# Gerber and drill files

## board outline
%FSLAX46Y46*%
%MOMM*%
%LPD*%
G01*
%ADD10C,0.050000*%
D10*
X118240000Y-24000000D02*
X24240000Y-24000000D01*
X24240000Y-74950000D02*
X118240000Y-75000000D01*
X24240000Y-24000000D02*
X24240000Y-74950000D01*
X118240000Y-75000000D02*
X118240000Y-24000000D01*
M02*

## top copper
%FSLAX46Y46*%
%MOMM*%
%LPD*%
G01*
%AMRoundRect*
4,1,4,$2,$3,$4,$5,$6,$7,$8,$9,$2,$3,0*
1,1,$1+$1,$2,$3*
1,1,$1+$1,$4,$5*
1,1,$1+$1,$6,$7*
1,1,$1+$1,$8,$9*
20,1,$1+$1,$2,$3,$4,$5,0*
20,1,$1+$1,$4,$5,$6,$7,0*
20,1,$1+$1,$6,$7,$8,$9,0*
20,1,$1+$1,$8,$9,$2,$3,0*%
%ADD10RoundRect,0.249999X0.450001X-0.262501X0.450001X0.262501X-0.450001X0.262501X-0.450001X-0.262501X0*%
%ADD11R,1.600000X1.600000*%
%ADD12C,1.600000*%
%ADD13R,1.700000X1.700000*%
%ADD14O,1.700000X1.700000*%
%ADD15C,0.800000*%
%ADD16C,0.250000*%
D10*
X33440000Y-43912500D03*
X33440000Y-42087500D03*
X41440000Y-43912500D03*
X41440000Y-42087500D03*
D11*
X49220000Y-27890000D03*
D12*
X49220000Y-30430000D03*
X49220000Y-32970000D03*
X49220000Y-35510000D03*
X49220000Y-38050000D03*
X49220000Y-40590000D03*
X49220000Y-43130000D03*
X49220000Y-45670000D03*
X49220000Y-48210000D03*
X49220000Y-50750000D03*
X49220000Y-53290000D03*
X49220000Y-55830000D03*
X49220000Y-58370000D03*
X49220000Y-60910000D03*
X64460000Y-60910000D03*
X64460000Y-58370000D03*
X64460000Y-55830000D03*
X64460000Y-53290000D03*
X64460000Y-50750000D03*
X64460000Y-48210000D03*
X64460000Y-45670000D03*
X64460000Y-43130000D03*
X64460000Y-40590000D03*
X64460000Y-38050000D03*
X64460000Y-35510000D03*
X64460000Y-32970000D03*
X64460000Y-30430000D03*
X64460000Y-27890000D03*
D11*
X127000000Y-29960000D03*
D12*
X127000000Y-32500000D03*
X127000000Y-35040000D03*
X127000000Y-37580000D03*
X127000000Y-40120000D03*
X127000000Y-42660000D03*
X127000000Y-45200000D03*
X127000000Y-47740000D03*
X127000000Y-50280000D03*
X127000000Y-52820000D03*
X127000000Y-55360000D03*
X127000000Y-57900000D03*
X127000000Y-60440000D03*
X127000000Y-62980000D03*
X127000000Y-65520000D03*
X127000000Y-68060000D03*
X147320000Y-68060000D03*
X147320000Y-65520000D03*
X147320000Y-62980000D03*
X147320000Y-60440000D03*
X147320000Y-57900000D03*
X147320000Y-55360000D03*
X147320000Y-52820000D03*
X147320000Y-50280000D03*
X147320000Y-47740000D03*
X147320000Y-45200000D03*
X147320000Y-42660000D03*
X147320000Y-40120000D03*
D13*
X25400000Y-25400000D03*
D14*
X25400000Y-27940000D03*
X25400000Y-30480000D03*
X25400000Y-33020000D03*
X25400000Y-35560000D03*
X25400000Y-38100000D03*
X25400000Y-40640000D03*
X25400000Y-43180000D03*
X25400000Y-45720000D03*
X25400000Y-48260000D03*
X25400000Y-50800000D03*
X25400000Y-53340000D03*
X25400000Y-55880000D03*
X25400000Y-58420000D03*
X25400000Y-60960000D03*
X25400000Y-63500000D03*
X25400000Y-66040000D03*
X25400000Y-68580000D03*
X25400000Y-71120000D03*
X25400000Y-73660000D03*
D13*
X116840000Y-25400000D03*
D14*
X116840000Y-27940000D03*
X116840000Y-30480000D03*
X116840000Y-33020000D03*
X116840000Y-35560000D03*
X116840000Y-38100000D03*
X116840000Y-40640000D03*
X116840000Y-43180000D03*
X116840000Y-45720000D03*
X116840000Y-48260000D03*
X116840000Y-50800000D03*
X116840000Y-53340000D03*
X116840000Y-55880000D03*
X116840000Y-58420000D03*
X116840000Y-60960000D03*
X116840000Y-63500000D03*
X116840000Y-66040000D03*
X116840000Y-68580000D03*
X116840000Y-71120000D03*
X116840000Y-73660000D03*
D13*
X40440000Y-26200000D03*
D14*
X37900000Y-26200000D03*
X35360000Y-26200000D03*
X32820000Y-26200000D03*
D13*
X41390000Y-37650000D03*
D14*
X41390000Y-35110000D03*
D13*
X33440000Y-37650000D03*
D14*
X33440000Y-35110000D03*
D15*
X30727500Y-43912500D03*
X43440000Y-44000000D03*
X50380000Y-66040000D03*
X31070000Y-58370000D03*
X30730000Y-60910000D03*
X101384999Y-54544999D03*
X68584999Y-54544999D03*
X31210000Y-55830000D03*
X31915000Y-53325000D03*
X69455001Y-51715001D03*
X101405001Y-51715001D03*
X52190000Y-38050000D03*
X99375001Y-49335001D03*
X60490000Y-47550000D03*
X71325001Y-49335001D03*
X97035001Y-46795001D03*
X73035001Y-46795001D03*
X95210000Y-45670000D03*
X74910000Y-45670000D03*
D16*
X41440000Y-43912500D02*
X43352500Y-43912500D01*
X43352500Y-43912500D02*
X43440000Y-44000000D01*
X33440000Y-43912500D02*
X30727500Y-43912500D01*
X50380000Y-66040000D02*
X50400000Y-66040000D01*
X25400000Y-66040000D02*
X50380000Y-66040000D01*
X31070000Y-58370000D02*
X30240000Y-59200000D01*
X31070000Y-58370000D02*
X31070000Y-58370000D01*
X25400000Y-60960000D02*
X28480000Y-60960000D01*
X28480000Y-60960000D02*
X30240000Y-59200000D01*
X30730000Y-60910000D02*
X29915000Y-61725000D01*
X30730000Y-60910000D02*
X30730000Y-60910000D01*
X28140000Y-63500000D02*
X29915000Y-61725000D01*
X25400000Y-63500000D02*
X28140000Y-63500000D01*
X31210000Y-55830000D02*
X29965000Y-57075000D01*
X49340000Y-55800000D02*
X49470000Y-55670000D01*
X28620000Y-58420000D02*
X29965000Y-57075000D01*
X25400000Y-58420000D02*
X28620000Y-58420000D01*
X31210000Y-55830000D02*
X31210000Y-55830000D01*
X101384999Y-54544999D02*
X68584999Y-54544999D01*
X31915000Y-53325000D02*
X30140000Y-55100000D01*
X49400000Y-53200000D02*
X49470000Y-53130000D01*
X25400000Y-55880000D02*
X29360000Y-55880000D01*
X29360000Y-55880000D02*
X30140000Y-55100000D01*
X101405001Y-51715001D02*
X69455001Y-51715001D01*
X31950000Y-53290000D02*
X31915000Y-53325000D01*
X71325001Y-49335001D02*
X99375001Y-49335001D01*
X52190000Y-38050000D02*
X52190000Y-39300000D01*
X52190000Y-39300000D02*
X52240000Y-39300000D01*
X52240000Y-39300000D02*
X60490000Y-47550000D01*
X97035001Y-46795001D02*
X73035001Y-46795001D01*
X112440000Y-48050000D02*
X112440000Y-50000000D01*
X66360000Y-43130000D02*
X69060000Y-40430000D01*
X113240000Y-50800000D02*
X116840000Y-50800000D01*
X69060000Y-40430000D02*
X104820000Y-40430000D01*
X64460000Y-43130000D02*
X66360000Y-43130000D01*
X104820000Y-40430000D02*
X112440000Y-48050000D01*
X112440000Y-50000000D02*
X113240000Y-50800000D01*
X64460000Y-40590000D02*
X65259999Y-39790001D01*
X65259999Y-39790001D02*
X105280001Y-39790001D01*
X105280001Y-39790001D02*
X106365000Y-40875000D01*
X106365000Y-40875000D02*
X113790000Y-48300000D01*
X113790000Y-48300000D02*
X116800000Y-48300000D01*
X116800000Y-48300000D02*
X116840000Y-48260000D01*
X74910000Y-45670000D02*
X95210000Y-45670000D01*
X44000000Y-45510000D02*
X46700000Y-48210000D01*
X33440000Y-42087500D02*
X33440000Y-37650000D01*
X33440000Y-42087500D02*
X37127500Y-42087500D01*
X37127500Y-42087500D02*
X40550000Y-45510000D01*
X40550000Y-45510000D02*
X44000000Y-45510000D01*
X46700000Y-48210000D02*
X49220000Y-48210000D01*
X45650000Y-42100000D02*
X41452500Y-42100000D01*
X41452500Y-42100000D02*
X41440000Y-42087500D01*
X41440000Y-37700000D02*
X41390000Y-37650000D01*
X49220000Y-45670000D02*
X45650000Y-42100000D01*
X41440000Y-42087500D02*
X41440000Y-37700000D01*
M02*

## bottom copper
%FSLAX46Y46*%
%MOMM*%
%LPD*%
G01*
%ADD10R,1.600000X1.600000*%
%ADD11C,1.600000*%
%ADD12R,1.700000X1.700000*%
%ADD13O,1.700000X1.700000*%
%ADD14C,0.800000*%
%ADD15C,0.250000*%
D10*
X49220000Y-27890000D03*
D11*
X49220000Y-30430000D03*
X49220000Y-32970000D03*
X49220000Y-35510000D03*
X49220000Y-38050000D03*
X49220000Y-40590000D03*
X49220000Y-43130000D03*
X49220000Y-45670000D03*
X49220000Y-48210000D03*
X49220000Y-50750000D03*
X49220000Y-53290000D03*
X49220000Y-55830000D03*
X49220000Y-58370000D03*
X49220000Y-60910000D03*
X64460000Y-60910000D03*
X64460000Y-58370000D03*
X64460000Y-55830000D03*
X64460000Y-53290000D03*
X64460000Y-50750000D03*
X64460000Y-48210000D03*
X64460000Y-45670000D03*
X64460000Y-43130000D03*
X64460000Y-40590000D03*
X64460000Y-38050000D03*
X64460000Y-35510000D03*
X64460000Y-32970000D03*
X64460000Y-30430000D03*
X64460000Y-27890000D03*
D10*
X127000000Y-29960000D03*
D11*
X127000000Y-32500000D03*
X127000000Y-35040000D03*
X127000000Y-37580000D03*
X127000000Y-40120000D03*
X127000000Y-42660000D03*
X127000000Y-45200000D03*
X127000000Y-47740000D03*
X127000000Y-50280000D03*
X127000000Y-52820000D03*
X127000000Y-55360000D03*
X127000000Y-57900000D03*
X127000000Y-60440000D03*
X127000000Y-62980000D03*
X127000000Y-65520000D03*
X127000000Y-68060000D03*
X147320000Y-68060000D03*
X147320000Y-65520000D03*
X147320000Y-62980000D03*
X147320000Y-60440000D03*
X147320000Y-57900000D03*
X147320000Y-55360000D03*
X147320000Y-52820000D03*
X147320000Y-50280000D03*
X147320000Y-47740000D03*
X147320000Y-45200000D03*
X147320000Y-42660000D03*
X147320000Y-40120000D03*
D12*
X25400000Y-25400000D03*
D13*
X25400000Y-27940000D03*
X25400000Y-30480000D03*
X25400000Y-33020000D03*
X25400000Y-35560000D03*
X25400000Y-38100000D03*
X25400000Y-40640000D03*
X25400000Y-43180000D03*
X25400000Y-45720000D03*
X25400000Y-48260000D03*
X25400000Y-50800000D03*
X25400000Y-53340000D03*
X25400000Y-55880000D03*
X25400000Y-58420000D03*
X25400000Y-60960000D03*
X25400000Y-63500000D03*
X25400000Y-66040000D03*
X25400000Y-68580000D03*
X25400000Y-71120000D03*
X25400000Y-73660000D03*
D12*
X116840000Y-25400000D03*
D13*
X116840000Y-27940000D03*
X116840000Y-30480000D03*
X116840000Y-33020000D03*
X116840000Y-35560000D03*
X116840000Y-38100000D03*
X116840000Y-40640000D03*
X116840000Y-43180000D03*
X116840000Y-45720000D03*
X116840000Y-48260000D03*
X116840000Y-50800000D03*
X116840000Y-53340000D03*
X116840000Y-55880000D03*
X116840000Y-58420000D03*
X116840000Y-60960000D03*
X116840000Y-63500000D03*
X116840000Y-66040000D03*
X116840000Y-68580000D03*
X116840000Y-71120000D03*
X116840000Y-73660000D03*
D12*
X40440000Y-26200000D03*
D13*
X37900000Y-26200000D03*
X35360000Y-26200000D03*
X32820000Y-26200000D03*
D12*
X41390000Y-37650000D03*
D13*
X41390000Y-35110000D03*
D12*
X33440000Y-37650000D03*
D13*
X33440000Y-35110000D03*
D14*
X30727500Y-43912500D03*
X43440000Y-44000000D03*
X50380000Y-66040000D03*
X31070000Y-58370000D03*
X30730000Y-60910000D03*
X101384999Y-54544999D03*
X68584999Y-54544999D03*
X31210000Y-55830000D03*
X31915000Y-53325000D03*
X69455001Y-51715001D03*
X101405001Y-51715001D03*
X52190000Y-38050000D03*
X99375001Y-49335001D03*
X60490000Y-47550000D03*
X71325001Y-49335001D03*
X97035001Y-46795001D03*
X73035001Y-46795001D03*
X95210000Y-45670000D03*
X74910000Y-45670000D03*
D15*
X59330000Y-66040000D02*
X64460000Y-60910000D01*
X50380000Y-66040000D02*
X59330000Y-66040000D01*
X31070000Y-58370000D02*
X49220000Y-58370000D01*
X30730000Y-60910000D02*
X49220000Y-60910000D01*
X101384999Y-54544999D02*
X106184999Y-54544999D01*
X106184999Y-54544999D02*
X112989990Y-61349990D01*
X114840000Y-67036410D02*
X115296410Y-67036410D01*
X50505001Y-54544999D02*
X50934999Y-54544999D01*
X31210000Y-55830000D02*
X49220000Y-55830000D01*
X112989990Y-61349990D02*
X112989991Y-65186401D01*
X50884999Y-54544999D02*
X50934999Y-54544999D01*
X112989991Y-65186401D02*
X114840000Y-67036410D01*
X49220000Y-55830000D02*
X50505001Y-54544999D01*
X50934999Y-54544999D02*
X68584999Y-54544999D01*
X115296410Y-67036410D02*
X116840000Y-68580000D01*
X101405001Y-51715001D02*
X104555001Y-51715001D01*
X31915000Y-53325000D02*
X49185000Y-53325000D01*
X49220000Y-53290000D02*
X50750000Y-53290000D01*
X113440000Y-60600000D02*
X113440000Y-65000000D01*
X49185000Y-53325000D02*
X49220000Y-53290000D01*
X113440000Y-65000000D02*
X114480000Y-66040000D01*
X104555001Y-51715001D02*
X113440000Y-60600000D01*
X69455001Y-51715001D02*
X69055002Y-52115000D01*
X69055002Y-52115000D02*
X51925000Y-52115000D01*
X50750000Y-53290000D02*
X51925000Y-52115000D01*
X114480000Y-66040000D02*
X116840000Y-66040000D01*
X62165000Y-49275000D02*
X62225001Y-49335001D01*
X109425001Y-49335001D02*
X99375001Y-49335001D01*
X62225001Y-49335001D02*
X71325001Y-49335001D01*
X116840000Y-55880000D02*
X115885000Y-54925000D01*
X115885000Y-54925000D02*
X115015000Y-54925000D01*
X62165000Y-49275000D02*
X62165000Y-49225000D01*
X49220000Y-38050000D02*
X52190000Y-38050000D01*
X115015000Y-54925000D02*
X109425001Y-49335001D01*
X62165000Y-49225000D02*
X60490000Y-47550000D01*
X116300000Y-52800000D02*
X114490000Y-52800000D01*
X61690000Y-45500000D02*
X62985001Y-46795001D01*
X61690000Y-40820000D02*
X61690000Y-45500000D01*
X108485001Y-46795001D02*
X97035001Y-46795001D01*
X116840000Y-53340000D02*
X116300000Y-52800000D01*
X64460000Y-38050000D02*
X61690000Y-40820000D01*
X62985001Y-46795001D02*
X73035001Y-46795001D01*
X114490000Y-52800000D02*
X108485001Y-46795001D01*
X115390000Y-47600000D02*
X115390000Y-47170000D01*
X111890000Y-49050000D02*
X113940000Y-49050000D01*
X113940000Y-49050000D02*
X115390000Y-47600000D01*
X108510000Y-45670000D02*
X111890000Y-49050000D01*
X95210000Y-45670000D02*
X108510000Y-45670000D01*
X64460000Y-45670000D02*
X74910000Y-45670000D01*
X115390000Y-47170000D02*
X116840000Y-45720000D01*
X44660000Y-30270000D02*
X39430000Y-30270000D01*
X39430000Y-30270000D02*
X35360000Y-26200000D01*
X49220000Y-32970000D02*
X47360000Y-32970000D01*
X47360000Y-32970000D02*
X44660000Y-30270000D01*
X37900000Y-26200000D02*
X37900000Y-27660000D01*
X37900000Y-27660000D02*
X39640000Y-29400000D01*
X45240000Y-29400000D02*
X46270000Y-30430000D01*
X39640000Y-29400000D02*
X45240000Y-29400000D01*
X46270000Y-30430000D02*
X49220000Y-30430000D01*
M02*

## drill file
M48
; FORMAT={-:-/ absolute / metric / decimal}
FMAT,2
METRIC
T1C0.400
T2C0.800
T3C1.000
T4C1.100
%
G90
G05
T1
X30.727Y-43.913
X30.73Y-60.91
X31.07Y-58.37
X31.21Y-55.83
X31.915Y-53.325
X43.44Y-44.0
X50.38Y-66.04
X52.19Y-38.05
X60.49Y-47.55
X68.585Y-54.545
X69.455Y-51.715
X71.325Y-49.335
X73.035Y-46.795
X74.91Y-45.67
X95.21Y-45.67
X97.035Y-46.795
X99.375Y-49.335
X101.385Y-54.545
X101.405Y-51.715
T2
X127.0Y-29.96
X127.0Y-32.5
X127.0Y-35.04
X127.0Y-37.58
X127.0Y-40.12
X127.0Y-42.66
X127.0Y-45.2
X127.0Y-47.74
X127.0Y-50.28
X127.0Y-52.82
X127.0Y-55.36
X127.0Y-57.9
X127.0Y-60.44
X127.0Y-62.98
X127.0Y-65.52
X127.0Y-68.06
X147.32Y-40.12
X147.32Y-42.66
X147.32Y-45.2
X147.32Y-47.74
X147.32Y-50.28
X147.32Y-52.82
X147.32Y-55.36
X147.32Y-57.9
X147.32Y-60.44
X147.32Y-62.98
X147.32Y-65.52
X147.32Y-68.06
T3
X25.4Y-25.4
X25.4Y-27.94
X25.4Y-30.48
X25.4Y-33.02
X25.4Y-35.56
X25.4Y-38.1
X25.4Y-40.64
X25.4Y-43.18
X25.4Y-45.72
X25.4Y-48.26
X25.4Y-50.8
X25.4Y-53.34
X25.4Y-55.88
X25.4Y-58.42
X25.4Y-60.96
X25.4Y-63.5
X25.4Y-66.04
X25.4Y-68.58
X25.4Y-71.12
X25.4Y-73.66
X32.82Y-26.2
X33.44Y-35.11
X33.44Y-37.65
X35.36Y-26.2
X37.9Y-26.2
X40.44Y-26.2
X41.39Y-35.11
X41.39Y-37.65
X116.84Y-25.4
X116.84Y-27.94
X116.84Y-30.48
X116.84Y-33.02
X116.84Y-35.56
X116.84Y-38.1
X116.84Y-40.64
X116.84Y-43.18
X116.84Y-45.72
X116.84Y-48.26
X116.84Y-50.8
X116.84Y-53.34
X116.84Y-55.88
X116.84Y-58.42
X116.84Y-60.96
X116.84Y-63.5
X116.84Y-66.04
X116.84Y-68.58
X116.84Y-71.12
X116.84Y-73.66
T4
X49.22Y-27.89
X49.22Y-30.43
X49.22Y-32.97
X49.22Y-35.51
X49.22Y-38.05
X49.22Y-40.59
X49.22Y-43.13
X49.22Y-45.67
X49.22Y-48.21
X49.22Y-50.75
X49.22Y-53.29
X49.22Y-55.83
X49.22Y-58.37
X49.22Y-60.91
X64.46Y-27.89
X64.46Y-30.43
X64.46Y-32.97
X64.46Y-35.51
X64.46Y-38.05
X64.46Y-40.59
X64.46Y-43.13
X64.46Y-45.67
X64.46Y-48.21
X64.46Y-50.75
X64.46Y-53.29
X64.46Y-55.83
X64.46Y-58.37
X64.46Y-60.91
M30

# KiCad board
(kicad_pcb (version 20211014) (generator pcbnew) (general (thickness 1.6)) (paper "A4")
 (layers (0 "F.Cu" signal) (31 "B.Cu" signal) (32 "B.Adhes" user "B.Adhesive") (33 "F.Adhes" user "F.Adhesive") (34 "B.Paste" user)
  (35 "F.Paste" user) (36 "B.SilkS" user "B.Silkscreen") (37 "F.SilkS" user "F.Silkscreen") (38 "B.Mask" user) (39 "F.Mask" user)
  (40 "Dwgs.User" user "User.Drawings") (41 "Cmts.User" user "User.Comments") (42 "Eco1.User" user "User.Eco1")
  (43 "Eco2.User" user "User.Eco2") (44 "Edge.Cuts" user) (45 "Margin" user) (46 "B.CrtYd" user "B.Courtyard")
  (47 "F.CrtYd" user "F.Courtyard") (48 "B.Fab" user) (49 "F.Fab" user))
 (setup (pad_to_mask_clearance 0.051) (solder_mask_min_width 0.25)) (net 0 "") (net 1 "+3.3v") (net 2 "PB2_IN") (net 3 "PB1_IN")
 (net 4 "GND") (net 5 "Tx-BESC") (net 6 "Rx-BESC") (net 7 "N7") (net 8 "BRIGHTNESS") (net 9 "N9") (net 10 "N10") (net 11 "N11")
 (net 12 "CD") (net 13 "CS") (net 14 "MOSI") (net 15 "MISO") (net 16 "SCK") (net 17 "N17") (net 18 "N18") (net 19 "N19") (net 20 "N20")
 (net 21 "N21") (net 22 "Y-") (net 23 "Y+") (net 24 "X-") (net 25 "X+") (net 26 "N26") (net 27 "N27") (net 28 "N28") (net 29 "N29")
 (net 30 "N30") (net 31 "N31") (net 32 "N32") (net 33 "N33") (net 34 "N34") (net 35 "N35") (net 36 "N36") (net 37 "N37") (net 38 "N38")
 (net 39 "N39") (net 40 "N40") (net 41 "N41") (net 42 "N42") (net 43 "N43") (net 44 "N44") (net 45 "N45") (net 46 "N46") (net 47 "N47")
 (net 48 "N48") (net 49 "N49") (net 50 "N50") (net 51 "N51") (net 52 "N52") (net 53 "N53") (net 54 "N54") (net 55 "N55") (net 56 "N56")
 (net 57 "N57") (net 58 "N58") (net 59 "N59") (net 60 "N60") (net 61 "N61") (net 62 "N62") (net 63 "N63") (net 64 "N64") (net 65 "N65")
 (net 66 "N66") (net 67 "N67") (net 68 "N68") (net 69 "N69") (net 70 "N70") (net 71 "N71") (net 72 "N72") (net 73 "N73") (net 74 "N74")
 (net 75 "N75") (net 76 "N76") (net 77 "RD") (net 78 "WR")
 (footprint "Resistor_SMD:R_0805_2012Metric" (layer "F.Cu") (at 33.44 43 90)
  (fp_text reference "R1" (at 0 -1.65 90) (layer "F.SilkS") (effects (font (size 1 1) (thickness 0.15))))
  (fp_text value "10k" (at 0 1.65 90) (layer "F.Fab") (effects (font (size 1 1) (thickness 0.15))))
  (pad "1" smd roundrect locked (at -0.9125 0 90) (size 1.025 1.4) (layers "F.Cu" "F.Paste" "F.Mask") (roundrect_rratio 0.2439014634)
   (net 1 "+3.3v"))
  (pad "2" smd roundrect locked (at 0.9125 0 90) (size 1.025 1.4) (layers "F.Cu" "F.Paste" "F.Mask") (roundrect_rratio 0.2439014634)
   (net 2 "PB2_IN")))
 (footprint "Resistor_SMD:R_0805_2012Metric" (layer "F.Cu") (at 41.44 43 90)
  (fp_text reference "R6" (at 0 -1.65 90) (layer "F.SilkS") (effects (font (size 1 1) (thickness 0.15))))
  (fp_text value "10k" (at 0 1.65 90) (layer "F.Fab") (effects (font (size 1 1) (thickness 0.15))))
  (pad "1" smd roundrect locked (at -0.9125 0 90) (size 1.025 1.4) (layers "F.Cu" "F.Paste" "F.Mask") (roundrect_rratio 0.2439014634)
   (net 1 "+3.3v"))
  (pad "2" smd roundrect locked (at 0.9125 0 90) (size 1.025 1.4) (layers "F.Cu" "F.Paste" "F.Mask") (roundrect_rratio 0.2439014634)
   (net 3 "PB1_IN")))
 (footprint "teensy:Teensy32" (layer "F.Cu") (at 56.84 44.4 -90)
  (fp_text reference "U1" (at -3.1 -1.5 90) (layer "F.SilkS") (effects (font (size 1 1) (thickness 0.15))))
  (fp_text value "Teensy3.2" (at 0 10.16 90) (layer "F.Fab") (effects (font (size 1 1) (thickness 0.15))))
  (pad "1" thru_hole rect locked (at -16.51 7.62 270) (size 1.6 1.6) (drill 1.1) (layers *.Cu *.Mask) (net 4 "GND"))
  (pad "2" thru_hole circle locked (at -13.97 7.62 270) (size 1.6 1.6) (drill 1.1) (layers *.Cu *.Mask) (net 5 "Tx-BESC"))
  (pad "3" thru_hole circle locked (at -11.43 7.62 270) (size 1.6 1.6) (drill 1.1) (layers *.Cu *.Mask) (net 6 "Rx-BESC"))
  (pad "4" thru_hole circle locked (at -8.89 7.62 270) (size 1.6 1.6) (drill 1.1) (layers *.Cu *.Mask) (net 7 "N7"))
  (pad "5" thru_hole circle locked (at -6.35 7.62 270) (size 1.6 1.6) (drill 1.1) (layers *.Cu *.Mask) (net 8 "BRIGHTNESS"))
  (pad "6" thru_hole circle locked (at -3.81 7.62 270) (size 1.6 1.6) (drill 1.1) (layers *.Cu *.Mask) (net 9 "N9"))
  (pad "7" thru_hole circle locked (at -1.27 7.62 270) (size 1.6 1.6) (drill 1.1) (layers *.Cu *.Mask) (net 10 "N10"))
  (pad "8" thru_hole circle locked (at 1.27 7.62 270) (size 1.6 1.6) (drill 1.1) (layers *.Cu *.Mask) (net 3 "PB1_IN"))
  (pad "9" thru_hole circle locked (at 3.81 7.62 270) (size 1.6 1.6) (drill 1.1) (layers *.Cu *.Mask) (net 2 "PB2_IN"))
  (pad "10" thru_hole circle locked (at 6.35 7.62 270) (size 1.6 1.6) (drill 1.1) (layers *.Cu *.Mask) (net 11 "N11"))
  (pad "11" thru_hole circle locked (at 8.89 7.62 270) (size 1.6 1.6) (drill 1.1) (layers *.Cu *.Mask) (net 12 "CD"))
  (pad "12" thru_hole circle locked (at 11.43 7.62 270) (size 1.6 1.6) (drill 1.1) (layers *.Cu *.Mask) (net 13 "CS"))
  (pad "13" thru_hole circle locked (at 13.97 7.62 270) (size 1.6 1.6) (drill 1.1) (layers *.Cu *.Mask) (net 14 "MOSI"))
  (pad "14" thru_hole circle locked (at 16.51 7.62 270) (size 1.6 1.6) (drill 1.1) (layers *.Cu *.Mask) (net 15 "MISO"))
  (pad "20" thru_hole circle locked (at 16.51 -7.62 270) (size 1.6 1.6) (drill 1.1) (layers *.Cu *.Mask) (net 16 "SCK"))
  (pad "21" thru_hole circle locked (at 13.97 -7.62 270) (size 1.6 1.6) (drill 1.1) (layers *.Cu *.Mask) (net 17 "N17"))
  (pad "22" thru_hole circle locked (at 11.43 -7.62 270) (size 1.6 1.6) (drill 1.1) (layers *.Cu *.Mask) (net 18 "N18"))
  (pad "23" thru_hole circle locked (at 8.89 -7.62 270) (size 1.6 1.6) (drill 1.1) (layers *.Cu *.Mask) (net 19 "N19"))
  (pad "24" thru_hole circle locked (at 6.35 -7.62 270) (size 1.6 1.6) (drill 1.1) (layers *.Cu *.Mask) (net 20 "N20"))
  (pad "25" thru_hole circle locked (at 3.81 -7.62 270) (size 1.6 1.6) (drill 1.1) (layers *.Cu *.Mask) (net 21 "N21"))
  (pad "26" thru_hole circle locked (at 1.27 -7.62 270) (size 1.6 1.6) (drill 1.1) (layers *.Cu *.Mask) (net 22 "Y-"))
  (pad "27" thru_hole circle locked (at -1.27 -7.62 270) (size 1.6 1.6) (drill 1.1) (layers *.Cu *.Mask) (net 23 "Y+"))
  (pad "28" thru_hole circle locked (at -3.81 -7.62 270) (size 1.6 1.6) (drill 1.1) (layers *.Cu *.Mask) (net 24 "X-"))
  (pad "29" thru_hole circle locked (at -6.35 -7.62 270) (size 1.6 1.6) (drill 1.1) (layers *.Cu *.Mask) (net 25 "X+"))
  (pad "30" thru_hole circle locked (at -8.89 -7.62 270) (size 1.6 1.6) (drill 1.1) (layers *.Cu *.Mask) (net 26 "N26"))
  (pad "31" thru_hole circle locked (at -11.43 -7.62 270) (size 1.6 1.6) (drill 1.1) (layers *.Cu *.Mask) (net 1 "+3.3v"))
  (pad "32" thru_hole circle locked (at -13.97 -7.62 270) (size 1.6 1.6) (drill 1.1) (layers *.Cu *.Mask) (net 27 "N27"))
  (pad "33" thru_hole circle locked (at -16.51 -7.62 270) (size 1.6 1.6) (drill 1.1) (layers *.Cu *.Mask) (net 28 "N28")))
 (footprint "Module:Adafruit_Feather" (layer "F.Cu") (at 127 29.96)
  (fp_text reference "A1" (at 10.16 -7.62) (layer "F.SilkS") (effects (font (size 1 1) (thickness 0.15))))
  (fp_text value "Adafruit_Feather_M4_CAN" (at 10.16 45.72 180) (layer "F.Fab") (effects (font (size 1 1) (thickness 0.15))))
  (pad "1" thru_hole rect (at 0 0 180) (size 1.6 1.6) (drill 0.8) (layers *.Cu *.Mask) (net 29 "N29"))
  (pad "2" thru_hole circle (at 0 2.54 180) (size 1.6 1.6) (drill 0.8) (layers *.Cu *.Mask) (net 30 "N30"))
  (pad "3" thru_hole circle (at 0 5.08 180) (size 1.6 1.6) (drill 0.8) (layers *.Cu *.Mask) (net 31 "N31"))
  (pad "4" thru_hole circle (at 0 7.62 180) (size 1.6 1.6) (drill 0.8) (layers *.Cu *.Mask) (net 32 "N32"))
  (pad "5" thru_hole circle (at 0 10.16 180) (size 1.6 1.6) (drill 0.8) (layers *.Cu *.Mask) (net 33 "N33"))
  (pad "6" thru_hole circle (at 0 12.7 180) (size 1.6 1.6) (drill 0.8) (layers *.Cu *.Mask) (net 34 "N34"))
  (pad "7" thru_hole circle (at 0 15.24 180) (size 1.6 1.6) (drill 0.8) (layers *.Cu *.Mask) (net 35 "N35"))
  (pad "8" thru_hole circle (at 0 17.78 180) (size 1.6 1.6) (drill 0.8) (layers *.Cu *.Mask) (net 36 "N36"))
  (pad "9" thru_hole circle (at 0 20.32 180) (size 1.6 1.6) (drill 0.8) (layers *.Cu *.Mask) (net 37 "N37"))
  (pad "10" thru_hole circle (at 0 22.86 180) (size 1.6 1.6) (drill 0.8) (layers *.Cu *.Mask) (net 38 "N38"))
  (pad "11" thru_hole circle (at 0 25.4 180) (size 1.6 1.6) (drill 0.8) (layers *.Cu *.Mask) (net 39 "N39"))
  (pad "12" thru_hole circle (at 0 27.94 180) (size 1.6 1.6) (drill 0.8) (layers *.Cu *.Mask) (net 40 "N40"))
  (pad "13" thru_hole circle (at 0 30.48 180) (size 1.6 1.6) (drill 0.8) (layers *.Cu *.Mask) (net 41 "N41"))
  (pad "14" thru_hole circle (at 0 33.02 180) (size 1.6 1.6) (drill 0.8) (layers *.Cu *.Mask) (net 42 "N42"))
  (pad "15" thru_hole circle (at 0 35.56 180) (size 1.6 1.6) (drill 0.8) (layers *.Cu *.Mask) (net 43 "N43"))
  (pad "16" thru_hole circle (at 0 38.1 180) (size 1.6 1.6) (drill 0.8) (layers *.Cu *.Mask) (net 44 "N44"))
  (pad "17" thru_hole circle (at 20.32 38.1 180) (size 1.6 1.6) (drill 0.8) (layers *.Cu *.Mask) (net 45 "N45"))
  (pad "18" thru_hole circle (at 20.32 35.56 180) (size 1.6 1.6) (drill 0.8) (layers *.Cu *.Mask) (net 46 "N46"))
  (pad "19" thru_hole circle (at 20.32 33.02 180) (size 1.6 1.6) (drill 0.8) (layers *.Cu *.Mask) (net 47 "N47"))
  (pad "20" thru_hole circle (at 20.32 30.48 180) (size 1.6 1.6) (drill 0.8) (layers *.Cu *.Mask) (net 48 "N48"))
  (pad "21" thru_hole circle (at 20.32 27.94 180) (size 1.6 1.6) (drill 0.8) (layers *.Cu *.Mask) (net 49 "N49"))
  (pad "22" thru_hole circle (at 20.32 25.4 180) (size 1.6 1.6) (drill 0.8) (layers *.Cu *.Mask) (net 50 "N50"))
  (pad "23" thru_hole circle (at 20.32 22.86 180) (size 1.6 1.6) (drill 0.8) (layers *.Cu *.Mask) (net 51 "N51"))
  (pad "24" thru_hole circle (at 20.32 20.32 180) (size 1.6 1.6) (drill 0.8) (layers *.Cu *.Mask) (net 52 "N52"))
  (pad "25" thru_hole circle (at 20.32 17.78 180) (size 1.6 1.6) (drill 0.8) (layers *.Cu *.Mask) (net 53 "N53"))
  (pad "26" thru_hole circle (at 20.32 15.24 180) (size 1.6 1.6) (drill 0.8) (layers *.Cu *.Mask) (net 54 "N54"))
  (pad "27" thru_hole circle (at 20.32 12.7 180) (size 1.6 1.6) (drill 0.8) (layers *.Cu *.Mask) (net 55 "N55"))
  (pad "28" thru_hole circle (at 20.32 10.16 180) (size 1.6 1.6) (drill 0.8) (layers *.Cu *.Mask) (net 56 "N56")))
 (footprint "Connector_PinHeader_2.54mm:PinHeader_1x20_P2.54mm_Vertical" (layer "B.Cu") (at 25.4 25.4 180)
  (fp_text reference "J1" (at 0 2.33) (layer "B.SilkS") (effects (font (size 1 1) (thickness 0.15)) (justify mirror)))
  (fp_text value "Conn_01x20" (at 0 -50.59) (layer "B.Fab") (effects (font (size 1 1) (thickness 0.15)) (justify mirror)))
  (pad "1" thru_hole rect locked (at 0 0 180) (size 1.7 1.7) (drill 1) (layers *.Cu *.Mask) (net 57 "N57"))
  (pad "2" thru_hole oval locked (at 0 -2.54 180) (size 1.7 1.7) (drill 1) (layers *.Cu *.Mask) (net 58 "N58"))
  (pad "3" thru_hole oval locked (at 0 -5.08 180) (size 1.7 1.7) (drill 1) (layers *.Cu *.Mask) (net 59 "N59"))
  (pad "4" thru_hole oval locked (at 0 -7.62 180) (size 1.7 1.7) (drill 1) (layers *.Cu *.Mask) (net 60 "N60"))
  (pad "5" thru_hole oval locked (at 0 -10.16 180) (size 1.7 1.7) (drill 1) (layers *.Cu *.Mask) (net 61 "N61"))
  (pad "6" thru_hole oval locked (at 0 -12.7 180) (size 1.7 1.7) (drill 1) (layers *.Cu *.Mask) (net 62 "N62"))
  (pad "7" thru_hole oval locked (at 0 -15.24 180) (size 1.7 1.7) (drill 1) (layers *.Cu *.Mask) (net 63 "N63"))
  (pad "8" thru_hole oval locked (at 0 -17.78 180) (size 1.7 1.7) (drill 1) (layers *.Cu *.Mask) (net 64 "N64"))
  (pad "9" thru_hole oval locked (at 0 -20.32 180) (size 1.7 1.7) (drill 1) (layers *.Cu *.Mask) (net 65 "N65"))
  (pad "10" thru_hole oval locked (at 0 -22.86 180) (size 1.7 1.7) (drill 1) (layers *.Cu *.Mask) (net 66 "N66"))
  (pad "11" thru_hole oval locked (at 0 -25.4 180) (size 1.7 1.7) (drill 1) (layers *.Cu *.Mask) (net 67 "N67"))
  (pad "12" thru_hole oval locked (at 0 -27.94 180) (size 1.7 1.7) (drill 1) (layers *.Cu *.Mask) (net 1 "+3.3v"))
  (pad "13" thru_hole oval locked (at 0 -30.48 180) (size 1.7 1.7) (drill 1) (layers *.Cu *.Mask) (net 12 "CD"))
  (pad "14" thru_hole oval locked (at 0 -33.02 180) (size 1.7 1.7) (drill 1) (layers *.Cu *.Mask) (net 13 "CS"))
  (pad "15" thru_hole oval locked (at 0 -35.56 180) (size 1.7 1.7) (drill 1) (layers *.Cu *.Mask) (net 14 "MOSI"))
  (pad "16" thru_hole oval locked (at 0 -38.1 180) (size 1.7 1.7) (drill 1) (layers *.Cu *.Mask) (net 15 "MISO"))
  (pad "17" thru_hole oval locked (at 0 -40.64 180) (size 1.7 1.7) (drill 1) (layers *.Cu *.Mask) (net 16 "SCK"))
  (pad "18" thru_hole oval locked (at 0 -43.18 180) (size 1.7 1.7) (drill 1) (layers *.Cu *.Mask) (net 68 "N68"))
  (pad "19" thru_hole oval locked (at 0 -45.72 180) (size 1.7 1.7) (drill 1) (layers *.Cu *.Mask) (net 1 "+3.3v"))
  (pad "20" thru_hole oval locked (at 0 -48.26 180) (size 1.7 1.7) (drill 1) (layers *.Cu *.Mask) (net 4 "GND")))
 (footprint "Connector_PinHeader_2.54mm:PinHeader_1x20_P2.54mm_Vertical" (layer "B.Cu") (at 116.84 25.4 180)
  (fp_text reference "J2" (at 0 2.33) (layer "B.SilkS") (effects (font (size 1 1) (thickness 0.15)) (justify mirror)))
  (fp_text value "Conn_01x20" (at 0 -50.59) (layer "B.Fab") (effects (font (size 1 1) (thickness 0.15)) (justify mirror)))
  (pad "1" thru_hole rect locked (at 0 0 180) (size 1.7 1.7) (drill 1) (layers *.Cu *.Mask) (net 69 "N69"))
  (pad "2" thru_hole oval locked (at 0 -2.54 180) (size 1.7 1.7) (drill 1) (layers *.Cu *.Mask) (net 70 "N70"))
  (pad "3" thru_hole oval locked (at 0 -5.08 180) (size 1.7 1.7) (drill 1) (layers *.Cu *.Mask) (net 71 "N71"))
  (pad "4" thru_hole oval locked (at 0 -7.62 180) (size 1.7 1.7) (drill 1) (layers *.Cu *.Mask) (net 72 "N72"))
  (pad "5" thru_hole oval locked (at 0 -10.16 180) (size 1.7 1.7) (drill 1) (layers *.Cu *.Mask) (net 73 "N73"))
  (pad "6" thru_hole oval locked (at 0 -12.7 180) (size 1.7 1.7) (drill 1) (layers *.Cu *.Mask) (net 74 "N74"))
  (pad "7" thru_hole oval locked (at 0 -15.24 180) (size 1.7 1.7) (drill 1) (layers *.Cu *.Mask) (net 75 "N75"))
  (pad "8" thru_hole oval locked (at 0 -17.78 180) (size 1.7 1.7) (drill 1) (layers *.Cu *.Mask) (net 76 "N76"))
  (pad "9" thru_hole oval locked (at 0 -20.32 180) (size 1.7 1.7) (drill 1) (layers *.Cu *.Mask) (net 22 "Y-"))
  (pad "10" thru_hole oval locked (at 0 -22.86 180) (size 1.7 1.7) (drill 1) (layers *.Cu *.Mask) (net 24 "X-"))
  (pad "11" thru_hole oval locked (at 0 -25.4 180) (size 1.7 1.7) (drill 1) (layers *.Cu *.Mask) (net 23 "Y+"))
  (pad "12" thru_hole oval locked (at 0 -27.94 180) (size 1.7 1.7) (drill 1) (layers *.Cu *.Mask) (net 25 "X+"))
  (pad "13" thru_hole oval locked (at 0 -30.48 180) (size 1.7 1.7) (drill 1) (layers *.Cu *.Mask) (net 8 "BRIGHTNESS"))
  (pad "14" thru_hole oval locked (at 0 -33.02 180) (size 1.7 1.7) (drill 1) (layers *.Cu *.Mask) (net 1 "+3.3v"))
  (pad "15" thru_hole oval locked (at 0 -35.56 180) (size 1.7 1.7) (drill 1) (layers *.Cu *.Mask) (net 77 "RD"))
  (pad "16" thru_hole oval locked (at 0 -38.1 180) (size 1.7 1.7) (drill 1) (layers *.Cu *.Mask) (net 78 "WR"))
  (pad "17" thru_hole oval locked (at 0 -40.64 180) (size 1.7 1.7) (drill 1) (layers *.Cu *.Mask) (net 12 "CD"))
  (pad "18" thru_hole oval locked (at 0 -43.18 180) (size 1.7 1.7) (drill 1) (layers *.Cu *.Mask) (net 13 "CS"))
  (pad "19" thru_hole oval locked (at 0 -45.72 180) (size 1.7 1.7) (drill 1) (layers *.Cu *.Mask) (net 1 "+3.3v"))
  (pad "20" thru_hole oval locked (at 0 -48.26 180) (size 1.7 1.7) (drill 1) (layers *.Cu *.Mask) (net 4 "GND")))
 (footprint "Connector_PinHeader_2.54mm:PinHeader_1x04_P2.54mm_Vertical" (layer "B.Cu") (at 40.44 26.2 90)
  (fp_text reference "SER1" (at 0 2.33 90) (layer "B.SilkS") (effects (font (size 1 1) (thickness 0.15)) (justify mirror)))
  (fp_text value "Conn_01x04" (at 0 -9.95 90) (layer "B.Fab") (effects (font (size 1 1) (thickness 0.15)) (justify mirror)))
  (pad "1" thru_hole rect locked (at 0 0 90) (size 1.7 1.7) (drill 1) (layers *.Cu *.Mask) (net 1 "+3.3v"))
  (pad "2" thru_hole oval locked (at 0 -2.54 90) (size 1.7 1.7) (drill 1) (layers *.Cu *.Mask) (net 5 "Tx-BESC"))
  (pad "3" thru_hole oval locked (at 0 -5.08 90) (size 1.7 1.7) (drill 1) (layers *.Cu *.Mask) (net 6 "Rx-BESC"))
  (pad "4" thru_hole oval locked (at 0 -7.62 90) (size 1.7 1.7) (drill 1) (layers *.Cu *.Mask) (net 4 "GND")))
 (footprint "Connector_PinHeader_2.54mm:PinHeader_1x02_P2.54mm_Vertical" (layer "B.Cu") (at 41.39 37.65)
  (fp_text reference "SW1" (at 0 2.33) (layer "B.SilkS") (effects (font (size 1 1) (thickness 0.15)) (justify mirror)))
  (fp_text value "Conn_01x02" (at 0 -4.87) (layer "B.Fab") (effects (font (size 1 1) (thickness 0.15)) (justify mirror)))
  (pad "1" thru_hole rect locked (at 0 0) (size 1.7 1.7) (drill 1) (layers *.Cu *.Mask) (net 3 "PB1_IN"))
  (pad "2" thru_hole oval locked (at 0 -2.54) (size 1.7 1.7) (drill 1) (layers *.Cu *.Mask) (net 4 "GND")))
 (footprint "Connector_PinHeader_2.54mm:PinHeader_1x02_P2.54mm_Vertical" (layer "B.Cu") (at 33.44 37.65)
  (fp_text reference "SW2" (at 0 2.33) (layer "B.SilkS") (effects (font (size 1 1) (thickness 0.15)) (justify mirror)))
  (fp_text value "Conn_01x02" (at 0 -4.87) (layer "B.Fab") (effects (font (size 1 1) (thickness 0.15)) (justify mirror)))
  (pad "1" thru_hole rect locked (at 0 0) (size 1.7 1.7) (drill 1) (layers *.Cu *.Mask) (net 2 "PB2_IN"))
  (pad "2" thru_hole oval locked (at 0 -2.54) (size 1.7 1.7) (drill 1) (layers *.Cu *.Mask) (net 4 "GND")))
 (gr_line (start 118.24 24) (end 24.24 24) (layer "Edge.Cuts") (width 0.05))
 (gr_line (start 24.24 74.95) (end 118.24 75) (layer "Edge.Cuts") (width 0.05))
 (gr_line (start 24.24 24) (end 24.24 74.95) (layer "Edge.Cuts") (width 0.05))
 (gr_line (start 118.24 75) (end 118.24 24) (layer "Edge.Cuts") (width 0.05))
 (segment (start 41.44 43.9125) (end 43.3525 43.9125) (width 0.25) (layer "F.Cu") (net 1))
 (segment (start 43.3525 43.9125) (end 43.44 44) (width 0.25) (layer "F.Cu") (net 1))
 (segment (start 33.44 43.9125) (end 30.7275 43.9125) (width 0.25) (layer "F.Cu") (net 1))
 (via (at 30.7275 43.9125) (size 0.8) (drill 0.4) (layers "F.Cu" "B.Cu") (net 1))
 (via (at 43.44 44) (size 0.8) (drill 0.4) (layers "F.Cu" "B.Cu") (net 1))
 (segment (start 50.38 66.04) (end 50.4 66.04) (width 0.25) (layer "F.Cu") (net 16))
 (segment (start 25.4 66.04) (end 50.38 66.04) (width 0.25) (layer "F.Cu") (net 16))
 (via (at 50.38 66.04) (size 0.8) (drill 0.4) (layers "F.Cu" "B.Cu") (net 16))
 (segment (start 59.33 66.04) (end 64.46 60.91) (width 0.25) (layer "B.Cu") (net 16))
 (segment (start 50.38 66.04) (end 59.33 66.04) (width 0.25) (layer "B.Cu") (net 16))
 (segment (start 31.07 58.37) (end 30.24 59.2) (width 0.25) (layer "F.Cu") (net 14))
 (segment (start 31.07 58.37) (end 31.07 58.37) (width 0.25) (layer "F.Cu") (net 14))
 (segment (start 25.4 60.96) (end 28.48 60.96) (width 0.25) (layer "F.Cu") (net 14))
 (segment (start 28.48 60.96) (end 30.24 59.2) (width 0.25) (layer "F.Cu") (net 14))
 (via (at 31.07 58.37) (size 0.8) (drill 0.4) (layers "F.Cu" "B.Cu") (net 14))
 (segment (start 31.07 58.37) (end 49.22 58.37) (width 0.25) (layer "B.Cu") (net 14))
 (segment (start 30.73 60.91) (end 29.915 61.725) (width 0.25) (layer "F.Cu") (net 15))
 (segment (start 30.73 60.91) (end 30.73 60.91) (width 0.25) (layer "F.Cu") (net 15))
 (segment (start 28.14 63.5) (end 29.915 61.725) (width 0.25) (layer "F.Cu") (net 15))
 (segment (start 25.4 63.5) (end 28.14 63.5) (width 0.25) (layer "F.Cu") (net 15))
 (via (at 30.73 60.91) (size 0.8) (drill 0.4) (layers "F.Cu" "B.Cu") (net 15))
 (segment (start 30.73 60.91) (end 49.22 60.91) (width 0.25) (layer "B.Cu") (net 15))
 (segment (start 31.21 55.83) (end 29.965 57.075) (width 0.25) (layer "F.Cu") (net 13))
 (segment (start 49.34 55.8) (end 49.47 55.67) (width 0.25) (layer "F.Cu") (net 13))
 (segment (start 28.62 58.42) (end 29.965 57.075) (width 0.25) (layer "F.Cu") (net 13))
 (segment (start 25.4 58.42) (end 28.62 58.42) (width 0.25) (layer "F.Cu") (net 13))
 (segment (start 31.21 55.83) (end 31.21 55.83) (width 0.25) (layer "F.Cu") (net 13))
 (segment (start 101.384999 54.544999) (end 68.584999 54.544999) (width 0.25) (layer "F.Cu") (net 13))
 (via (at 101.384999 54.544999) (size 0.8) (drill 0.4) (layers "F.Cu" "B.Cu") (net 13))
 (via (at 68.584999 54.544999) (size 0.8) (drill 0.4) (layers "F.Cu" "B.Cu") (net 13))
 (via (at 31.21 55.83) (size 0.8) (drill 0.4) (layers "F.Cu" "B.Cu") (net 13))
 (segment (start 101.384999 54.544999) (end 106.184999 54.544999) (width 0.25) (layer "B.Cu") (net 13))
 (segment (start 106.184999 54.544999) (end 112.98999 61.34999) (width 0.25) (layer "B.Cu") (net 13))
 (segment (start 114.84 67.03641) (end 115.29641 67.03641) (width 0.25) (layer "B.Cu") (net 13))
 (segment (start 50.505001 54.544999) (end 50.934999 54.544999) (width 0.25) (layer "B.Cu") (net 13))
 (segment (start 31.21 55.83) (end 49.22 55.83) (width 0.25) (layer "B.Cu") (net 13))
 (segment (start 112.98999 61.34999) (end 112.989991 65.186401) (width 0.25) (layer "B.Cu") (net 13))
 (segment (start 50.884999 54.544999) (end 50.934999 54.544999) (width 0.25) (layer "B.Cu") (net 13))
 (segment (start 112.989991 65.186401) (end 114.84 67.03641) (width 0.25) (layer "B.Cu") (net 13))
 (segment (start 49.22 55.83) (end 50.505001 54.544999) (width 0.25) (layer "B.Cu") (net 13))
 (segment (start 50.934999 54.544999) (end 68.584999 54.544999) (width 0.25) (layer "B.Cu") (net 13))
 (segment (start 115.29641 67.03641) (end 116.84 68.58) (width 0.25) (layer "B.Cu") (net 13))
 (segment (start 31.915 53.325) (end 30.14 55.1) (width 0.25) (layer "F.Cu") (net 12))
 (segment (start 49.4 53.2) (end 49.47 53.13) (width 0.25) (layer "F.Cu") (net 12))
 (segment (start 25.4 55.88) (end 29.36 55.88) (width 0.25) (layer "F.Cu") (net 12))
 (segment (start 29.36 55.88) (end 30.14 55.1) (width 0.25) (layer "F.Cu") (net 12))
 (segment (start 101.405001 51.715001) (end 69.455001 51.715001) (width 0.25) (layer "F.Cu") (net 12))
 (segment (start 31.95 53.29) (end 31.915 53.325) (width 0.25) (layer "F.Cu") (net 12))
 (via (at 31.915 53.325) (size 0.8) (drill 0.4) (layers "F.Cu" "B.Cu") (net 12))
 (via (at 69.455001 51.715001) (size 0.8) (drill 0.4) (layers "F.Cu" "B.Cu") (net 12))
 (via (at 101.405001 51.715001) (size 0.8) (drill 0.4) (layers "F.Cu" "B.Cu") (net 12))
 (segment (start 101.405001 51.715001) (end 104.555001 51.715001) (width 0.25) (layer "B.Cu") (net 12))
 (segment (start 31.915 53.325) (end 49.185 53.325) (width 0.25) (layer "B.Cu") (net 12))
 (segment (start 49.22 53.29) (end 50.75 53.29) (width 0.25) (layer "B.Cu") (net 12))
 (segment (start 113.44 60.6) (end 113.44 65) (width 0.25) (layer "B.Cu") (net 12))
 (segment (start 49.185 53.325) (end 49.22 53.29) (width 0.25) (layer "B.Cu") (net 12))
 (segment (start 113.44 65) (end 114.48 66.04) (width 0.25) (layer "B.Cu") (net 12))
 (segment (start 104.555001 51.715001) (end 113.44 60.6) (width 0.25) (layer "B.Cu") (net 12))
 (segment (start 69.455001 51.715001) (end 69.055002 52.115) (width 0.25) (layer "B.Cu") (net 12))
 (segment (start 69.055002 52.115) (end 51.925 52.115) (width 0.25) (layer "B.Cu") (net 12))
 (segment (start 50.75 53.29) (end 51.925 52.115) (width 0.25) (layer "B.Cu") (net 12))
 (segment (start 114.48 66.04) (end 116.84 66.04) (width 0.25) (layer "B.Cu") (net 12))
 (segment (start 71.325001 49.335001) (end 99.375001 49.335001) (width 0.25) (layer "F.Cu") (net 8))
 (segment (start 52.19 38.05) (end 52.19 39.3) (width 0.25) (layer "F.Cu") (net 8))
 (segment (start 52.19 39.3) (end 52.24 39.3) (width 0.25) (layer "F.Cu") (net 8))
 (segment (start 52.24 39.3) (end 60.49 47.55) (width 0.25) (layer "F.Cu") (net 8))
 (via (at 52.19 38.05) (size 0.8) (drill 0.4) (layers "F.Cu" "B.Cu") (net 8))
 (via (at 99.375001 49.335001) (size 0.8) (drill 0.4) (layers "F.Cu" "B.Cu") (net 8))
 (via (at 60.49 47.55) (size 0.8) (drill 0.4) (layers "F.Cu" "B.Cu") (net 8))
 (via (at 71.325001 49.335001) (size 0.8) (drill 0.4) (layers "F.Cu" "B.Cu") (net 8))
 (segment (start 62.165 49.275) (end 62.225001 49.335001) (width 0.25) (layer "B.Cu") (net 8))
 (segment (start 109.425001 49.335001) (end 99.375001 49.335001) (width 0.25) (layer "B.Cu") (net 8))
 (segment (start 62.225001 49.335001) (end 71.325001 49.335001) (width 0.25) (layer "B.Cu") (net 8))
 (segment (start 116.84 55.88) (end 115.885 54.925) (width 0.25) (layer "B.Cu") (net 8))
 (segment (start 115.885 54.925) (end 115.015 54.925) (width 0.25) (layer "B.Cu") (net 8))
 (segment (start 62.165 49.275) (end 62.165 49.225) (width 0.25) (layer "B.Cu") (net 8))
 (segment (start 49.22 38.05) (end 52.19 38.05) (width 0.25) (layer "B.Cu") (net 8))
 (segment (start 115.015 54.925) (end 109.425001 49.335001) (width 0.25) (layer "B.Cu") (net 8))
 (segment (start 62.165 49.225) (end 60.49 47.55) (width 0.25) (layer "B.Cu") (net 8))
 (segment (start 97.035001 46.795001) (end 73.035001 46.795001) (width 0.25) (layer "F.Cu") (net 25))
 (via (at 97.035001 46.795001) (size 0.8) (drill 0.4) (layers "F.Cu" "B.Cu") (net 25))
 (via (at 73.035001 46.795001) (size 0.8) (drill 0.4) (layers "F.Cu" "B.Cu") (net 25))
 (segment (start 116.3 52.8) (end 114.49 52.8) (width 0.25) (layer "B.Cu") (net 25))
 (segment (start 61.69 45.5) (end 62.985001 46.795001) (width 0.25) (layer "B.Cu") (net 25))
 (segment (start 61.69 40.82) (end 61.69 45.5) (width 0.25) (layer "B.Cu") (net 25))
 (segment (start 108.485001 46.795001) (end 97.035001 46.795001) (width 0.25) (layer "B.Cu") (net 25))
 (segment (start 116.84 53.34) (end 116.3 52.8) (width 0.25) (layer "B.Cu") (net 25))
 (segment (start 64.46 38.05) (end 61.69 40.82) (width 0.25) (layer "B.Cu") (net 25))
 (segment (start 62.985001 46.795001) (end 73.035001 46.795001) (width 0.25) (layer "B.Cu") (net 25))
 (segment (start 114.49 52.8) (end 108.485001 46.795001) (width 0.25) (layer "B.Cu") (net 25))
 (segment (start 112.44 48.05) (end 112.44 50) (width 0.25) (layer "F.Cu") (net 23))
 (segment (start 66.36 43.13) (end 69.06 40.43) (width 0.25) (layer "F.Cu") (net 23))
 (segment (start 113.24 50.8) (end 116.84 50.8) (width 0.25) (layer "F.Cu") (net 23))
 (segment (start 69.06 40.43) (end 104.82 40.43) (width 0.25) (layer "F.Cu") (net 23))
 (segment (start 64.46 43.13) (end 66.36 43.13) (width 0.25) (layer "F.Cu") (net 23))
 (segment (start 104.82 40.43) (end 112.44 48.05) (width 0.25) (layer "F.Cu") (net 23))
 (segment (start 112.44 50) (end 113.24 50.8) (width 0.25) (layer "F.Cu") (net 23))
 (segment (start 64.46 40.59) (end 65.259999 39.790001) (width 0.25) (layer "F.Cu") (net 24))
 (segment (start 65.259999 39.790001) (end 105.280001 39.790001) (width 0.25) (layer "F.Cu") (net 24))
 (segment (start 105.280001 39.790001) (end 106.365 40.875) (width 0.25) (layer "F.Cu") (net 24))
 (segment (start 106.365 40.875) (end 113.79 48.3) (width 0.25) (layer "F.Cu") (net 24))
 (segment (start 113.79 48.3) (end 116.8 48.3) (width 0.25) (layer "F.Cu") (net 24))
 (segment (start 116.8 48.3) (end 116.84 48.26) (width 0.25) (layer "F.Cu") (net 24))
 (segment (start 74.91 45.67) (end 95.21 45.67) (width 0.25) (layer "F.Cu") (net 22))
 (via (at 95.21 45.67) (size 0.8) (drill 0.4) (layers "F.Cu" "B.Cu") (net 22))
 (via (at 74.91 45.67) (size 0.8) (drill 0.4) (layers "F.Cu" "B.Cu") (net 22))
 (segment (start 115.39 47.6) (end 115.39 47.17) (width 0.25) (layer "B.Cu") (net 22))
 (segment (start 111.89 49.05) (end 113.94 49.05) (width 0.25) (layer "B.Cu") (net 22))
 (segment (start 113.94 49.05) (end 115.39 47.6) (width 0.25) (layer "B.Cu") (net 22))
 (segment (start 108.51 45.67) (end 111.89 49.05) (width 0.25) (layer "B.Cu") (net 22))
 (segment (start 95.21 45.67) (end 108.51 45.67) (width 0.25) (layer "B.Cu") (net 22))
 (segment (start 64.46 45.67) (end 74.91 45.67) (width 0.25) (layer "B.Cu") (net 22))
 (segment (start 115.39 47.17) (end 116.84 45.72) (width 0.25) (layer "B.Cu") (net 22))
 (segment (start 44 45.51) (end 46.7 48.21) (width 0.25) (layer "F.Cu") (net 2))
 (segment (start 33.44 42.0875) (end 33.44 37.65) (width 0.25) (layer "F.Cu") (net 2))
 (segment (start 33.44 42.0875) (end 37.1275 42.0875) (width 0.25) (layer "F.Cu") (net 2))
 (segment (start 37.1275 42.0875) (end 40.55 45.51) (width 0.25) (layer "F.Cu") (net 2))
 (segment (start 40.55 45.51) (end 44 45.51) (width 0.25) (layer "F.Cu") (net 2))
 (segment (start 46.7 48.21) (end 49.22 48.21) (width 0.25) (layer "F.Cu") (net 2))
 (segment (start 45.65 42.1) (end 41.4525 42.1) (width 0.25) (layer "F.Cu") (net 3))
 (segment (start 41.4525 42.1) (end 41.44 42.0875) (width 0.25) (layer "F.Cu") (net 3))
 (segment (start 41.44 37.7) (end 41.39 37.65) (width 0.25) (layer "F.Cu") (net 3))
 (segment (start 49.22 45.67) (end 45.65 42.1) (width 0.25) (layer "F.Cu") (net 3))
 (segment (start 41.44 42.0875) (end 41.44 37.7) (width 0.25) (layer "F.Cu") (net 3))
 (segment (start 44.66 30.27) (end 39.43 30.27) (width 0.25) (layer "B.Cu") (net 6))
 (segment (start 39.43 30.27) (end 35.36 26.2) (width 0.25) (layer "B.Cu") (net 6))
 (segment (start 49.22 32.97) (end 47.36 32.97) (width 0.25) (layer "B.Cu") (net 6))
 (segment (start 47.36 32.97) (end 44.66 30.27) (width 0.25) (layer "B.Cu") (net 6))
 (segment (start 37.9 26.2) (end 37.9 27.66) (width 0.25) (layer "B.Cu") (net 5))
 (segment (start 37.9 27.66) (end 39.64 29.4) (width 0.25) (layer "B.Cu") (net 5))
 (segment (start 45.24 29.4) (end 46.27 30.43) (width 0.25) (layer "B.Cu") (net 5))
 (segment (start 39.64 29.4) (end 45.24 29.4) (width 0.25) (layer "B.Cu") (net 5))
 (segment (start 46.27 30.43) (end 49.22 30.43) (width 0.25) (layer "B.Cu") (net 5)))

